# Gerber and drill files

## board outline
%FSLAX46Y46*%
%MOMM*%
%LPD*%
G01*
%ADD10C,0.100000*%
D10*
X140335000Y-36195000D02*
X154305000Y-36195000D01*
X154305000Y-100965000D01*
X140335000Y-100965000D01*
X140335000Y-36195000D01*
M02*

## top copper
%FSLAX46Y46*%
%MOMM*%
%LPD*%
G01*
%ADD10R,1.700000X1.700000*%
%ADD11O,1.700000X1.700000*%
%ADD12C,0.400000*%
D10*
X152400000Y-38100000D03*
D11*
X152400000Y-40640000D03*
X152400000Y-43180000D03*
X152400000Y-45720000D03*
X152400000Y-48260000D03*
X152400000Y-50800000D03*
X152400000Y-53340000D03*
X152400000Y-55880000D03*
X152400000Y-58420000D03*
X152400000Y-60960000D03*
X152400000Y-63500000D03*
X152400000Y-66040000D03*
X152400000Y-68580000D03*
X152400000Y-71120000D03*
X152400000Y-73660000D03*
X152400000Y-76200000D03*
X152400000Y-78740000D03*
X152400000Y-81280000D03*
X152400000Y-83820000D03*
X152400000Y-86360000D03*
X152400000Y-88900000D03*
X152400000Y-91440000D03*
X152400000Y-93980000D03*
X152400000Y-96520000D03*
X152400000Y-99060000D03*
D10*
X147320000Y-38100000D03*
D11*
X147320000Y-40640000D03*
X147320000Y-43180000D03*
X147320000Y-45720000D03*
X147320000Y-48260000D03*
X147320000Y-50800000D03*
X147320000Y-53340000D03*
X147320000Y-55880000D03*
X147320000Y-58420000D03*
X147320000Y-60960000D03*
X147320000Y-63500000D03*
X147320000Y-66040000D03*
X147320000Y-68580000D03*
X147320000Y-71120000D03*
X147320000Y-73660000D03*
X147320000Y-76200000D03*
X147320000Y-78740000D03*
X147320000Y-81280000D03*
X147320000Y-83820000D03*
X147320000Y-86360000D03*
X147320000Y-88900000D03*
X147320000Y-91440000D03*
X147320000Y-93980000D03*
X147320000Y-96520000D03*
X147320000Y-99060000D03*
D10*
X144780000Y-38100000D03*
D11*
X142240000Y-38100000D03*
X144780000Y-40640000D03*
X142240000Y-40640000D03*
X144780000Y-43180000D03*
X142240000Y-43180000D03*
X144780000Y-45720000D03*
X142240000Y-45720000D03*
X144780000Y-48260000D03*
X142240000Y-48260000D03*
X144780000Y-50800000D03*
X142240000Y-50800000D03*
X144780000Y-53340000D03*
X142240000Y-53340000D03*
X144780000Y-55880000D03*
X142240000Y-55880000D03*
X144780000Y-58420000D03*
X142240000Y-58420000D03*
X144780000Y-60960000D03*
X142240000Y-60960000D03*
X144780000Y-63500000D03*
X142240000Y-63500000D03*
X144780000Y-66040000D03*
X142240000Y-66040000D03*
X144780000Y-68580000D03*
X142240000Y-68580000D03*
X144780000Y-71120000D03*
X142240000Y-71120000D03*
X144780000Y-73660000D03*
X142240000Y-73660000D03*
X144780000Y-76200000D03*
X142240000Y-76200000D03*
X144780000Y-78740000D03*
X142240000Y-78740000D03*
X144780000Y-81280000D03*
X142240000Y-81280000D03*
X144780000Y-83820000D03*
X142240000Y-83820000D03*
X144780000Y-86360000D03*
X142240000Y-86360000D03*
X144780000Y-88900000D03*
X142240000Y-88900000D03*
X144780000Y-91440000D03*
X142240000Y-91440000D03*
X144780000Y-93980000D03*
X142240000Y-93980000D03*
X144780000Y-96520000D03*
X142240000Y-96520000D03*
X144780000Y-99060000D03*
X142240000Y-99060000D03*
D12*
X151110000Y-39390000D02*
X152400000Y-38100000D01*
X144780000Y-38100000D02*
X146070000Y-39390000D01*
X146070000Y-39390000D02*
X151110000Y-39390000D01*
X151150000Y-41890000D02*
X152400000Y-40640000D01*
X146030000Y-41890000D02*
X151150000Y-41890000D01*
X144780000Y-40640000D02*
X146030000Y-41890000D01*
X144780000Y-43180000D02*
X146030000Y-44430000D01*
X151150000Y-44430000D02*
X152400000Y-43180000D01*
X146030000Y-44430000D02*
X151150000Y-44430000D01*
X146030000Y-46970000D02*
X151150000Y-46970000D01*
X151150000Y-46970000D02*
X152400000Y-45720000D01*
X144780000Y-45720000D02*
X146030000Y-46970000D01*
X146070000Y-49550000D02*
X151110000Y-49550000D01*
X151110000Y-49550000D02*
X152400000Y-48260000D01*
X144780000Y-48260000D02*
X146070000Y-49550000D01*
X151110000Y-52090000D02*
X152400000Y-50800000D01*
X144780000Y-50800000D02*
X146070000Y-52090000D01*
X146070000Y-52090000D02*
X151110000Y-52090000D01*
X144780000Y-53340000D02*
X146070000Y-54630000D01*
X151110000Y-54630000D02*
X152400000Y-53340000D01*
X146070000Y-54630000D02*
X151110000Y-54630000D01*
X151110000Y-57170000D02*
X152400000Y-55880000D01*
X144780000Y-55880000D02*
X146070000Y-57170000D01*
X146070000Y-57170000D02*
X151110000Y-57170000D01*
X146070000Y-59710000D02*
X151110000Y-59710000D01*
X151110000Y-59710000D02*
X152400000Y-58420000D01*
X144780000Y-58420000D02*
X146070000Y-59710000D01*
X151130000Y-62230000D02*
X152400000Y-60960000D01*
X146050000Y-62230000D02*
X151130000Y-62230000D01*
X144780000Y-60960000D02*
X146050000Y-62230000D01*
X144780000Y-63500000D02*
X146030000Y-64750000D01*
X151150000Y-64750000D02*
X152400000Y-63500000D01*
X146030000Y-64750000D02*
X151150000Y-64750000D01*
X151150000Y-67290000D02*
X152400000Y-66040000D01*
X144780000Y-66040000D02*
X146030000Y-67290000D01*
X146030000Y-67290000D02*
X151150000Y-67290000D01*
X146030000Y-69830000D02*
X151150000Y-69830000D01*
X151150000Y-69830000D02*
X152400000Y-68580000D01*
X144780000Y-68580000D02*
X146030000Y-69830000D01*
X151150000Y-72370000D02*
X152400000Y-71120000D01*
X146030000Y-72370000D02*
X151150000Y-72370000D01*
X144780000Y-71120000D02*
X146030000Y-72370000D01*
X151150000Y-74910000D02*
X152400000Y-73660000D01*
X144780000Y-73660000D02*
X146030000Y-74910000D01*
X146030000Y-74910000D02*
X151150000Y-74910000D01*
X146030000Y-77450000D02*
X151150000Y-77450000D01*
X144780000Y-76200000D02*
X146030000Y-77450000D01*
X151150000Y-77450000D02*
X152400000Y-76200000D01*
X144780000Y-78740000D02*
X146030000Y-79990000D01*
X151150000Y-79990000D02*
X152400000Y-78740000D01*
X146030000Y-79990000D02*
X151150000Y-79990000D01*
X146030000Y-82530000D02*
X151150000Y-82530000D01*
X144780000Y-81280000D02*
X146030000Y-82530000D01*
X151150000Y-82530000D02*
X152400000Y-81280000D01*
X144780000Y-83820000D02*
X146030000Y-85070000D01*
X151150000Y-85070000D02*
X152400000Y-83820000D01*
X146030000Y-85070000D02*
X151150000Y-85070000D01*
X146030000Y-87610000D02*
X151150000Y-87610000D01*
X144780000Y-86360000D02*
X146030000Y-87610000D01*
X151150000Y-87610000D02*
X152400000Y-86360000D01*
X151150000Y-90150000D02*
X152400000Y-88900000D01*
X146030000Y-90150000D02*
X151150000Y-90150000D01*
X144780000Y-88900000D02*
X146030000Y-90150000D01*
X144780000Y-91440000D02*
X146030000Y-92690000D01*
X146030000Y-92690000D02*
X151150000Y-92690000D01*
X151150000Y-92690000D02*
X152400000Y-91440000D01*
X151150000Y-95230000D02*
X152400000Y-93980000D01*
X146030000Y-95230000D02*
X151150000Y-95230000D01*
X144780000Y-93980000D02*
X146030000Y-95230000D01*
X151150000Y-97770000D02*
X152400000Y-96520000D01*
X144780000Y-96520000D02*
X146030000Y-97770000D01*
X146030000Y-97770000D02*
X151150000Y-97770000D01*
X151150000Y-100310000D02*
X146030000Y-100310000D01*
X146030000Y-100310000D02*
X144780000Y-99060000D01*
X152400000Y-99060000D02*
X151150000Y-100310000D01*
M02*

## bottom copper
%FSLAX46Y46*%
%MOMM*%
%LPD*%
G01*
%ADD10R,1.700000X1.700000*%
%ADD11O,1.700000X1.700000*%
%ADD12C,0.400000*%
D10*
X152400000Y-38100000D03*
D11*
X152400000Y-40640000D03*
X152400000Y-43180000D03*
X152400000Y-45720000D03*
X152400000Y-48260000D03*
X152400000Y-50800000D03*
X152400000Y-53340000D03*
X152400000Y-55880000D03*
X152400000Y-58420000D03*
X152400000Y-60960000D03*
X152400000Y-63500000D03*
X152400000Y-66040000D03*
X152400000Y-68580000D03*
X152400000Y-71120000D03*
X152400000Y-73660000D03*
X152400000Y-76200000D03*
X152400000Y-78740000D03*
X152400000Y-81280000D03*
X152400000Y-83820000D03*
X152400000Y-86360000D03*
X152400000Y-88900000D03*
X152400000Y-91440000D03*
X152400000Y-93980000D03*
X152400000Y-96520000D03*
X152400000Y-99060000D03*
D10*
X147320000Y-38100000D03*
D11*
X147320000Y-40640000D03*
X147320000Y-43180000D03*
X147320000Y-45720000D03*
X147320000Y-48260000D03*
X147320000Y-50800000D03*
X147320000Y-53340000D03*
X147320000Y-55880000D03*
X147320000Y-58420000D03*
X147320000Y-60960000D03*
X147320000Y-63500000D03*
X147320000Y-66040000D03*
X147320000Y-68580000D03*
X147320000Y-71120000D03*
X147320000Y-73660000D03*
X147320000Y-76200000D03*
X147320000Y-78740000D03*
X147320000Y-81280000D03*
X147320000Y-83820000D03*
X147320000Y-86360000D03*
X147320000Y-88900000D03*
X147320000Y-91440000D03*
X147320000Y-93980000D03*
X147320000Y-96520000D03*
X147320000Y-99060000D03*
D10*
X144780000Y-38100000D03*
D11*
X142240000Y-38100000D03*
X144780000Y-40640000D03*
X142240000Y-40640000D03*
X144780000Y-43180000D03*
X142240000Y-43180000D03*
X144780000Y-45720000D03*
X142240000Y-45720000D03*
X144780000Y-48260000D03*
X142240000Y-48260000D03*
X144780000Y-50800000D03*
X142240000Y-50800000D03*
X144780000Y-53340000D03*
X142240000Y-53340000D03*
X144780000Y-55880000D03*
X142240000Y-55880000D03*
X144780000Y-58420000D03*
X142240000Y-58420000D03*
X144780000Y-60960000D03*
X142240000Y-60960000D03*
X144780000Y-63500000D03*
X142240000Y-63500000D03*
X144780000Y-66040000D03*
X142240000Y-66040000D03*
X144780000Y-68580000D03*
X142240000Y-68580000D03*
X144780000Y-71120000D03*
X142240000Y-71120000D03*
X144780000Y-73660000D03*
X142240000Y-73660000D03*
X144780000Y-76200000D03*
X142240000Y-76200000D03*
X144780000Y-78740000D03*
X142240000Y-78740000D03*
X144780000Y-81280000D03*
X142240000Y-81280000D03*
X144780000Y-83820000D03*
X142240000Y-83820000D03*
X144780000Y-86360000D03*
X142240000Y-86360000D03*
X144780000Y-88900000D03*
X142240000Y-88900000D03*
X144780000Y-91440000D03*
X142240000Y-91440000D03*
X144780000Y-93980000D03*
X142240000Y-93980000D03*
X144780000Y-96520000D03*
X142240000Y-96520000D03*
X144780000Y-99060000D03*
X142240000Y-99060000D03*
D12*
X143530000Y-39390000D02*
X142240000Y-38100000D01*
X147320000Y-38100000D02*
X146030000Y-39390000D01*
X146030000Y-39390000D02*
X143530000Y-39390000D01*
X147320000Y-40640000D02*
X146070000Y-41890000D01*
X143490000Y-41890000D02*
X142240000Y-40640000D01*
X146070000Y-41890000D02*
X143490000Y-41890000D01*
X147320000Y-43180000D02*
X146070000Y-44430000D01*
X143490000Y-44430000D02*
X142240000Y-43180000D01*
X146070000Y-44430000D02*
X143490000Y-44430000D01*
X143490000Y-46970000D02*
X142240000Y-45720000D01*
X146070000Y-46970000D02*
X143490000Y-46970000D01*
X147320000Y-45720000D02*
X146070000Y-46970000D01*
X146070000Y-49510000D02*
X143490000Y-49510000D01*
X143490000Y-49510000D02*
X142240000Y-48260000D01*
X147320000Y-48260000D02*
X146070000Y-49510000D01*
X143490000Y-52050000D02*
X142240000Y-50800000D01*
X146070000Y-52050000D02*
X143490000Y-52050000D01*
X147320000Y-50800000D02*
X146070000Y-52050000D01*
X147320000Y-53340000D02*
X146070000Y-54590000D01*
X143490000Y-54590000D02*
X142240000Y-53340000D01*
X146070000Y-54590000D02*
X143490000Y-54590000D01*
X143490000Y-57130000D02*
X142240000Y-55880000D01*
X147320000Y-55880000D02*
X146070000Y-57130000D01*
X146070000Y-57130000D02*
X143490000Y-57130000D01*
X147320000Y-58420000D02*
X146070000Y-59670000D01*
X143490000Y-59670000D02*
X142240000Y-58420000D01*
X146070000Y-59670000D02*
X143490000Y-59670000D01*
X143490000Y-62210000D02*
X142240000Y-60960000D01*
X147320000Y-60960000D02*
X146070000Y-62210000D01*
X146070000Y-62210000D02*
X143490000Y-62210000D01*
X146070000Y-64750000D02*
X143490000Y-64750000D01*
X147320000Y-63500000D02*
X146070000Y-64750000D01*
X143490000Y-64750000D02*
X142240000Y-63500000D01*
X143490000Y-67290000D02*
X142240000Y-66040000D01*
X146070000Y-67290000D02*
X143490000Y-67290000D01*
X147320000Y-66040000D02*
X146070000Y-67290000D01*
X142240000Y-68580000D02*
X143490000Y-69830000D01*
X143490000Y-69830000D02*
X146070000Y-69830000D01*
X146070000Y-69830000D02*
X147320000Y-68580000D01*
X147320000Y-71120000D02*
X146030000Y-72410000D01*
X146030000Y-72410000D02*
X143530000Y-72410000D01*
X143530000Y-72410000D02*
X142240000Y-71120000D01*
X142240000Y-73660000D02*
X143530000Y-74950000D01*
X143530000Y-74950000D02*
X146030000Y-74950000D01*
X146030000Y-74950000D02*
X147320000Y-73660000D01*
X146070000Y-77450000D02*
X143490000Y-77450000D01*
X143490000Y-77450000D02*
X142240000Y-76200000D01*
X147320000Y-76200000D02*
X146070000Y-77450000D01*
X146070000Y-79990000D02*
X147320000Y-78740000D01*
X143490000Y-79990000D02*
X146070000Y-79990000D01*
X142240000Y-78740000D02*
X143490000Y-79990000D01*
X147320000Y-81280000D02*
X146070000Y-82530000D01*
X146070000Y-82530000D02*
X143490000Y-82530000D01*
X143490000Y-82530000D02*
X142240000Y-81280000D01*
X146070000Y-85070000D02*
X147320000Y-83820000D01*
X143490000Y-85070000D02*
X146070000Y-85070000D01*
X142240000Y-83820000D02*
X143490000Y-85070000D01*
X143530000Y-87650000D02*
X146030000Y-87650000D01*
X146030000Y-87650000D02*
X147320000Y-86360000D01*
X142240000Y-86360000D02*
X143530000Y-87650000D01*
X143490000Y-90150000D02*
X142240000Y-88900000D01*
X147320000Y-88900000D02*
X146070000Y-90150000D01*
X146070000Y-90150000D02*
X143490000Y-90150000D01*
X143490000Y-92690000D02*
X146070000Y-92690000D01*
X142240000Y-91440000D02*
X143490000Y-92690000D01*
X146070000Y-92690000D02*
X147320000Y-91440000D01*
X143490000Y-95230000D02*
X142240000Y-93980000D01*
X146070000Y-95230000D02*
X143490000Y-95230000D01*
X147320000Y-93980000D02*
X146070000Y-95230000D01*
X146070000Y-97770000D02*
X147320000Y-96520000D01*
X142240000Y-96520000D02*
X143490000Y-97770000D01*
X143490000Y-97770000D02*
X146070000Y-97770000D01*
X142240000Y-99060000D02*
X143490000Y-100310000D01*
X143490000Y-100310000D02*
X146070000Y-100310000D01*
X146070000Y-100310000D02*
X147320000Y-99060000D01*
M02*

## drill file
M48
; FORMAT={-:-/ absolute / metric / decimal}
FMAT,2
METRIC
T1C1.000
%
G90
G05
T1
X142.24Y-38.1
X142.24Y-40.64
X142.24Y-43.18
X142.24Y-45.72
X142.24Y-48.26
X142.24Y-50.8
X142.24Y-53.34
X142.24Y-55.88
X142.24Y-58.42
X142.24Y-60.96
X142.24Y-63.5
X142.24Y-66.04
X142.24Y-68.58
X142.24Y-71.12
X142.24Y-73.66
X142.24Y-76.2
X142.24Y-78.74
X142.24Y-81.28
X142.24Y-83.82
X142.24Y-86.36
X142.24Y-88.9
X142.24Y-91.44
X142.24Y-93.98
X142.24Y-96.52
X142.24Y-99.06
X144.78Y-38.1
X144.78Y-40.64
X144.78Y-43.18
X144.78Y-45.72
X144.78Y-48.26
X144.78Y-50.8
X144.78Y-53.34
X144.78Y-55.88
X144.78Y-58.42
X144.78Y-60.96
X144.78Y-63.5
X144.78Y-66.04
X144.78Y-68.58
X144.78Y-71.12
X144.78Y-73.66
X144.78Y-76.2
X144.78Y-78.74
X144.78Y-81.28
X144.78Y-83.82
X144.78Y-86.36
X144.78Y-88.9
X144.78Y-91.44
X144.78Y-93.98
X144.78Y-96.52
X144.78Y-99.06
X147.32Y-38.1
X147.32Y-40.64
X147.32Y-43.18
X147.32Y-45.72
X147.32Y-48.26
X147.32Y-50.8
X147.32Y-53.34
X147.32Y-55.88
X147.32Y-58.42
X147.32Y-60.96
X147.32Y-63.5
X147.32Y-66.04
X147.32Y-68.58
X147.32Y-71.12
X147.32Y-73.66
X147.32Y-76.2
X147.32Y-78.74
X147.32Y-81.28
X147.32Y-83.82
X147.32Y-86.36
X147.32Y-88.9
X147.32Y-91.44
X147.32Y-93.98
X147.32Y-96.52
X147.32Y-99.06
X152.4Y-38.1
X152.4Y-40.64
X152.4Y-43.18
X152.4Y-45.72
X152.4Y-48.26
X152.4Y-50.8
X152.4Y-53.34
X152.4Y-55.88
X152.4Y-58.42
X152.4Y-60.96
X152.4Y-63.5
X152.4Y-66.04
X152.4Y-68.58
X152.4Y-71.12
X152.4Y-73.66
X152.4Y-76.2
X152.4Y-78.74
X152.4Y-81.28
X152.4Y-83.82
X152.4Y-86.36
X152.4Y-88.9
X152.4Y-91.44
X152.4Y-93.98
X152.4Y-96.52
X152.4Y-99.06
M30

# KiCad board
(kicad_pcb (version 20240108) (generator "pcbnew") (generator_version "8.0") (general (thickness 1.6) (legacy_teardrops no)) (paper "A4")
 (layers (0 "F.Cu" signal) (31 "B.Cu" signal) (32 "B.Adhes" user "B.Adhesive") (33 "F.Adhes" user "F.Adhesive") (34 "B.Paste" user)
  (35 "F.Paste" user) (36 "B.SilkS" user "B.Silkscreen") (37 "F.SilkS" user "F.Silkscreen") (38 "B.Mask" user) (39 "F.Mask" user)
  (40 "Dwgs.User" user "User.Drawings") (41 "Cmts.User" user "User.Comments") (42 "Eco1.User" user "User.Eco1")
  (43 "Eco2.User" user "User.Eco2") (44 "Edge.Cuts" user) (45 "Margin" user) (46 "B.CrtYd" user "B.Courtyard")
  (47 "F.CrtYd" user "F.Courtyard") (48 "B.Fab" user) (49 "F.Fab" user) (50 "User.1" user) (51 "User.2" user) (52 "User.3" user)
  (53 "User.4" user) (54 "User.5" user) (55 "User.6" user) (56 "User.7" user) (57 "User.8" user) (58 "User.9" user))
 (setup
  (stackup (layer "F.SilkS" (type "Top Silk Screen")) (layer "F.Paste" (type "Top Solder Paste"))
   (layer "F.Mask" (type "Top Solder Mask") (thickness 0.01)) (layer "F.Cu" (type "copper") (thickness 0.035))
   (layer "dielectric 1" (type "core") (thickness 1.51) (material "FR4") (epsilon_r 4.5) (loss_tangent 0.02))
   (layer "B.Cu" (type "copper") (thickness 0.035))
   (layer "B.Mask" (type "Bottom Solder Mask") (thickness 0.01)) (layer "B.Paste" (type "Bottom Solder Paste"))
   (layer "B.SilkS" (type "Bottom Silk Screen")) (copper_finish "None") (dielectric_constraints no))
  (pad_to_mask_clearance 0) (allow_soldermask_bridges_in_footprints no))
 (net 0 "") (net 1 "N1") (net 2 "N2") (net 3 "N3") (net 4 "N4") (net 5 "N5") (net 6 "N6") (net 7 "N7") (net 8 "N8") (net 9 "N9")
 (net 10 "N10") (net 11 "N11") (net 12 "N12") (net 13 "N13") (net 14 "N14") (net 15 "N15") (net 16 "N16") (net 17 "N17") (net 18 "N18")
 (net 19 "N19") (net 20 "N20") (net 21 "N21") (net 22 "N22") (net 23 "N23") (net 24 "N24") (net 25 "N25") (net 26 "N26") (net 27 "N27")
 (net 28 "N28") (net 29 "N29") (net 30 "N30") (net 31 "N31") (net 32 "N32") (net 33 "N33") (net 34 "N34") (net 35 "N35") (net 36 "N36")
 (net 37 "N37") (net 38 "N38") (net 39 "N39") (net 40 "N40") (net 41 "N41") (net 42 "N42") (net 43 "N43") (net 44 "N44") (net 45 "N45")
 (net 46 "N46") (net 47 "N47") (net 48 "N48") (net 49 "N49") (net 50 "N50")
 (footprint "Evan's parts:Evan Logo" (layer "F.Cu") (at 149.86 49.53 90)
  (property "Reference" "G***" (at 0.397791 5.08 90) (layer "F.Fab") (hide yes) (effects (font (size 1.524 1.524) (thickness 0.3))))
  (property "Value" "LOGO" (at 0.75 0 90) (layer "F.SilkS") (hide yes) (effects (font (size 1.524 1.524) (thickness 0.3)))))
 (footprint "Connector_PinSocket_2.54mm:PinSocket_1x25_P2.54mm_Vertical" (layer "F.Cu") (at 152.4 38.1)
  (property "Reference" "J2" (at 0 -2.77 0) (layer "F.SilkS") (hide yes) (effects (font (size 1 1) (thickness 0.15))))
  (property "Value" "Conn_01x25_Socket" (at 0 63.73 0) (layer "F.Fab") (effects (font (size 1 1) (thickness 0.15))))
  (pad "1" thru_hole rect (at 0 0) (size 1.7 1.7) (drill 1) (layers "*.Cu" "*.Mask") (remove_unused_layers no) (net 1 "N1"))
  (pad "2" thru_hole oval (at 0 2.54) (size 1.7 1.7) (drill 1) (layers "*.Cu" "*.Mask") (remove_unused_layers no) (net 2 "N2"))
  (pad "3" thru_hole oval (at 0 5.08) (size 1.7 1.7) (drill 1) (layers "*.Cu" "*.Mask") (remove_unused_layers no) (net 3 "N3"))
  (pad "4" thru_hole oval (at 0 7.62) (size 1.7 1.7) (drill 1) (layers "*.Cu" "*.Mask") (remove_unused_layers no) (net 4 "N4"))
  (pad "5" thru_hole oval (at 0 10.16) (size 1.7 1.7) (drill 1) (layers "*.Cu" "*.Mask") (remove_unused_layers no) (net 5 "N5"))
  (pad "6" thru_hole oval (at 0 12.7) (size 1.7 1.7) (drill 1) (layers "*.Cu" "*.Mask") (remove_unused_layers no) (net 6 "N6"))
  (pad "7" thru_hole oval (at 0 15.24) (size 1.7 1.7) (drill 1) (layers "*.Cu" "*.Mask") (remove_unused_layers no) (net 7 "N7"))
  (pad "8" thru_hole oval (at 0 17.78) (size 1.7 1.7) (drill 1) (layers "*.Cu" "*.Mask") (remove_unused_layers no) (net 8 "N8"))
  (pad "9" thru_hole oval (at 0 20.32) (size 1.7 1.7) (drill 1) (layers "*.Cu" "*.Mask") (remove_unused_layers no) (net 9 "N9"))
  (pad "10" thru_hole oval (at 0 22.86) (size 1.7 1.7) (drill 1) (layers "*.Cu" "*.Mask") (remove_unused_layers no) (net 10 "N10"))
  (pad "11" thru_hole oval (at 0 25.4) (size 1.7 1.7) (drill 1) (layers "*.Cu" "*.Mask") (remove_unused_layers no) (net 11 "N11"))
  (pad "12" thru_hole oval (at 0 27.94) (size 1.7 1.7) (drill 1) (layers "*.Cu" "*.Mask") (remove_unused_layers no) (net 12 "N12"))
  (pad "13" thru_hole oval (at 0 30.48) (size 1.7 1.7) (drill 1) (layers "*.Cu" "*.Mask") (remove_unused_layers no) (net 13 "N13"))
  (pad "14" thru_hole oval (at 0 33.02) (size 1.7 1.7) (drill 1) (layers "*.Cu" "*.Mask") (remove_unused_layers no) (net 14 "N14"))
  (pad "15" thru_hole oval (at 0 35.56) (size 1.7 1.7) (drill 1) (layers "*.Cu" "*.Mask") (remove_unused_layers no) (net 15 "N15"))
  (pad "16" thru_hole oval (at 0 38.1) (size 1.7 1.7) (drill 1) (layers "*.Cu" "*.Mask") (remove_unused_layers no) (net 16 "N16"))
  (pad "17" thru_hole oval (at 0 40.64) (size 1.7 1.7) (drill 1) (layers "*.Cu" "*.Mask") (remove_unused_layers no) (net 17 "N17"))
  (pad "18" thru_hole oval (at 0 43.18) (size 1.7 1.7) (drill 1) (layers "*.Cu" "*.Mask") (remove_unused_layers no) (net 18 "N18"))
  (pad "19" thru_hole oval (at 0 45.72) (size 1.7 1.7) (drill 1) (layers "*.Cu" "*.Mask") (remove_unused_layers no) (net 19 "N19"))
  (pad "20" thru_hole oval (at 0 48.26) (size 1.7 1.7) (drill 1) (layers "*.Cu" "*.Mask") (remove_unused_layers no) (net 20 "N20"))
  (pad "21" thru_hole oval (at 0 50.8) (size 1.7 1.7) (drill 1) (layers "*.Cu" "*.Mask") (remove_unused_layers no) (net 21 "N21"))
  (pad "22" thru_hole oval (at 0 53.34) (size 1.7 1.7) (drill 1) (layers "*.Cu" "*.Mask") (remove_unused_layers no) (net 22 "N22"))
  (pad "23" thru_hole oval (at 0 55.88) (size 1.7 1.7) (drill 1) (layers "*.Cu" "*.Mask") (remove_unused_layers no) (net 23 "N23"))
  (pad "24" thru_hole oval (at 0 58.42) (size 1.7 1.7) (drill 1) (layers "*.Cu" "*.Mask") (remove_unused_layers no) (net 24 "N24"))
  (pad "25" thru_hole oval (at 0 60.96) (size 1.7 1.7) (drill 1) (layers "*.Cu" "*.Mask") (remove_unused_layers no) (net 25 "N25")))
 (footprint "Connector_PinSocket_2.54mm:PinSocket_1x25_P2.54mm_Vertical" (layer "F.Cu") (at 147.32 38.1)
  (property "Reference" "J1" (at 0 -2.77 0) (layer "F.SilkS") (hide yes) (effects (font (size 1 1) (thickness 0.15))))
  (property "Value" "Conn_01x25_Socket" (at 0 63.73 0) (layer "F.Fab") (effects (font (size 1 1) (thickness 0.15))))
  (pad "1" thru_hole rect (at 0 0) (size 1.7 1.7) (drill 1) (layers "*.Cu" "*.Mask") (remove_unused_layers no) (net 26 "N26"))
  (pad "2" thru_hole oval (at 0 2.54) (size 1.7 1.7) (drill 1) (layers "*.Cu" "*.Mask") (remove_unused_layers no) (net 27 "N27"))
  (pad "3" thru_hole oval (at 0 5.08) (size 1.7 1.7) (drill 1) (layers "*.Cu" "*.Mask") (remove_unused_layers no) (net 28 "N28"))
  (pad "4" thru_hole oval (at 0 7.62) (size 1.7 1.7) (drill 1) (layers "*.Cu" "*.Mask") (remove_unused_layers no) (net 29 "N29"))
  (pad "5" thru_hole oval (at 0 10.16) (size 1.7 1.7) (drill 1) (layers "*.Cu" "*.Mask") (remove_unused_layers no) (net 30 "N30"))
  (pad "6" thru_hole oval (at 0 12.7) (size 1.7 1.7) (drill 1) (layers "*.Cu" "*.Mask") (remove_unused_layers no) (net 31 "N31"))
  (pad "7" thru_hole oval (at 0 15.24) (size 1.7 1.7) (drill 1) (layers "*.Cu" "*.Mask") (remove_unused_layers no) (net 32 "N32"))
  (pad "8" thru_hole oval (at 0 17.78) (size 1.7 1.7) (drill 1) (layers "*.Cu" "*.Mask") (remove_unused_layers no) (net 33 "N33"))
  (pad "9" thru_hole oval (at 0 20.32) (size 1.7 1.7) (drill 1) (layers "*.Cu" "*.Mask") (remove_unused_layers no) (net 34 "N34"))
  (pad "10" thru_hole oval (at 0 22.86) (size 1.7 1.7) (drill 1) (layers "*.Cu" "*.Mask") (remove_unused_layers no) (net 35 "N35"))
  (pad "11" thru_hole oval (at 0 25.4) (size 1.7 1.7) (drill 1) (layers "*.Cu" "*.Mask") (remove_unused_layers no) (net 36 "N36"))
  (pad "12" thru_hole oval (at 0 27.94) (size 1.7 1.7) (drill 1) (layers "*.Cu" "*.Mask") (remove_unused_layers no) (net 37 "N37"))
  (pad "13" thru_hole oval (at 0 30.48) (size 1.7 1.7) (drill 1) (layers "*.Cu" "*.Mask") (remove_unused_layers no) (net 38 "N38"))
  (pad "14" thru_hole oval (at 0 33.02) (size 1.7 1.7) (drill 1) (layers "*.Cu" "*.Mask") (remove_unused_layers no) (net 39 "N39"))
  (pad "15" thru_hole oval (at 0 35.56) (size 1.7 1.7) (drill 1) (layers "*.Cu" "*.Mask") (remove_unused_layers no) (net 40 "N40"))
  (pad "16" thru_hole oval (at 0 38.1) (size 1.7 1.7) (drill 1) (layers "*.Cu" "*.Mask") (remove_unused_layers no) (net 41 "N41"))
  (pad "17" thru_hole oval (at 0 40.64) (size 1.7 1.7) (drill 1) (layers "*.Cu" "*.Mask") (remove_unused_layers no) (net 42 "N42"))
  (pad "18" thru_hole oval (at 0 43.18) (size 1.7 1.7) (drill 1) (layers "*.Cu" "*.Mask") (remove_unused_layers no) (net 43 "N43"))
  (pad "19" thru_hole oval (at 0 45.72) (size 1.7 1.7) (drill 1) (layers "*.Cu" "*.Mask") (remove_unused_layers no) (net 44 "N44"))
  (pad "20" thru_hole oval (at 0 48.26) (size 1.7 1.7) (drill 1) (layers "*.Cu" "*.Mask") (remove_unused_layers no) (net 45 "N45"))
  (pad "21" thru_hole oval (at 0 50.8) (size 1.7 1.7) (drill 1) (layers "*.Cu" "*.Mask") (remove_unused_layers no) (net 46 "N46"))
  (pad "22" thru_hole oval (at 0 53.34) (size 1.7 1.7) (drill 1) (layers "*.Cu" "*.Mask") (remove_unused_layers no) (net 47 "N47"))
  (pad "23" thru_hole oval (at 0 55.88) (size 1.7 1.7) (drill 1) (layers "*.Cu" "*.Mask") (remove_unused_layers no) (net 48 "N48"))
  (pad "24" thru_hole oval (at 0 58.42) (size 1.7 1.7) (drill 1) (layers "*.Cu" "*.Mask") (remove_unused_layers no) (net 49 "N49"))
  (pad "25" thru_hole oval (at 0 60.96) (size 1.7 1.7) (drill 1) (layers "*.Cu" "*.Mask") (remove_unused_layers no) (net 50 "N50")))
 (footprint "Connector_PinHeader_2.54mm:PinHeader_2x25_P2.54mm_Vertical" (layer "B.Cu") (at 144.78 38.1 180)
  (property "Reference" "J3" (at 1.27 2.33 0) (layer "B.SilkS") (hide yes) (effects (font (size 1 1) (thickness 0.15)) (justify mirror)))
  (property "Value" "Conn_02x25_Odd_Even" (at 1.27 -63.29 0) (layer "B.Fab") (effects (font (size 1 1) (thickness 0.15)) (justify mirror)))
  (pad "1" thru_hole rect (at 0 0 180) (size 1.7 1.7) (drill 1) (layers "*.Cu" "*.Mask") (remove_unused_layers no) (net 1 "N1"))
  (pad "2" thru_hole oval (at 2.54 0 180) (size 1.7 1.7) (drill 1) (layers "*.Cu" "*.Mask") (remove_unused_layers no) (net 26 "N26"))
  (pad "3" thru_hole oval (at 0 -2.54 180) (size 1.7 1.7) (drill 1) (layers "*.Cu" "*.Mask") (remove_unused_layers no) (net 2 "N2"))
  (pad "4" thru_hole oval (at 2.54 -2.54 180) (size 1.7 1.7) (drill 1) (layers "*.Cu" "*.Mask") (remove_unused_layers no) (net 27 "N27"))
  (pad "5" thru_hole oval (at 0 -5.08 180) (size 1.7 1.7) (drill 1) (layers "*.Cu" "*.Mask") (remove_unused_layers no) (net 3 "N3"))
  (pad "6" thru_hole oval (at 2.54 -5.08 180) (size 1.7 1.7) (drill 1) (layers "*.Cu" "*.Mask") (remove_unused_layers no) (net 28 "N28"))
  (pad "7" thru_hole oval (at 0 -7.62 180) (size 1.7 1.7) (drill 1) (layers "*.Cu" "*.Mask") (remove_unused_layers no) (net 4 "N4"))
  (pad "8" thru_hole oval (at 2.54 -7.62 180) (size 1.7 1.7) (drill 1) (layers "*.Cu" "*.Mask") (remove_unused_layers no) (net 29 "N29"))
  (pad "9" thru_hole oval (at 0 -10.16 180) (size 1.7 1.7) (drill 1) (layers "*.Cu" "*.Mask") (remove_unused_layers no) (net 5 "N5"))
  (pad "10" thru_hole oval (at 2.54 -10.16 180) (size 1.7 1.7) (drill 1) (layers "*.Cu" "*.Mask") (remove_unused_layers no) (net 30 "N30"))
  (pad "11" thru_hole oval (at 0 -12.7 180) (size 1.7 1.7) (drill 1) (layers "*.Cu" "*.Mask") (remove_unused_layers no) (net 6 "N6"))
  (pad "12" thru_hole oval (at 2.54 -12.7 180) (size 1.7 1.7) (drill 1) (layers "*.Cu" "*.Mask") (remove_unused_layers no) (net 31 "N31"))
  (pad "13" thru_hole oval (at 0 -15.24 180) (size 1.7 1.7) (drill 1) (layers "*.Cu" "*.Mask") (remove_unused_layers no) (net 7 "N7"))
  (pad "14" thru_hole oval (at 2.54 -15.24 180) (size 1.7 1.7) (drill 1) (layers "*.Cu" "*.Mask") (remove_unused_layers no) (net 32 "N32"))
  (pad "15" thru_hole oval (at 0 -17.78 180) (size 1.7 1.7) (drill 1) (layers "*.Cu" "*.Mask") (remove_unused_layers no) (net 8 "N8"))
  (pad "16" thru_hole oval (at 2.54 -17.78 180) (size 1.7 1.7) (drill 1) (layers "*.Cu" "*.Mask") (remove_unused_layers no) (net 33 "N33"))
  (pad "17" thru_hole oval (at 0 -20.32 180) (size 1.7 1.7) (drill 1) (layers "*.Cu" "*.Mask") (remove_unused_layers no) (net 9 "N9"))
  (pad "18" thru_hole oval (at 2.54 -20.32 180) (size 1.7 1.7) (drill 1) (layers "*.Cu" "*.Mask") (remove_unused_layers no) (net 34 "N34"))
  (pad "19" thru_hole oval (at 0 -22.86 180) (size 1.7 1.7) (drill 1) (layers "*.Cu" "*.Mask") (remove_unused_layers no) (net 10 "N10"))
  (pad "20" thru_hole oval (at 2.54 -22.86 180) (size 1.7 1.7) (drill 1) (layers "*.Cu" "*.Mask") (remove_unused_layers no) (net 35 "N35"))
  (pad "21" thru_hole oval (at 0 -25.4 180) (size 1.7 1.7) (drill 1) (layers "*.Cu" "*.Mask") (remove_unused_layers no) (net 11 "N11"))
  (pad "22" thru_hole oval (at 2.54 -25.4 180) (size 1.7 1.7) (drill 1) (layers "*.Cu" "*.Mask") (remove_unused_layers no) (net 36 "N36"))
  (pad "23" thru_hole oval (at 0 -27.94 180) (size 1.7 1.7) (drill 1) (layers "*.Cu" "*.Mask") (remove_unused_layers no) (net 12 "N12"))
  (pad "24" thru_hole oval (at 2.54 -27.94 180) (size 1.7 1.7) (drill 1) (layers "*.Cu" "*.Mask") (remove_unused_layers no) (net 37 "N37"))
  (pad "25" thru_hole oval (at 0 -30.48 180) (size 1.7 1.7) (drill 1) (layers "*.Cu" "*.Mask") (remove_unused_layers no) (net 13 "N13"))
  (pad "26" thru_hole oval (at 2.54 -30.48 180) (size 1.7 1.7) (drill 1) (layers "*.Cu" "*.Mask") (remove_unused_layers no) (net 38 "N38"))
  (pad "27" thru_hole oval (at 0 -33.02 180) (size 1.7 1.7) (drill 1) (layers "*.Cu" "*.Mask") (remove_unused_layers no) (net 14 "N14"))
  (pad "28" thru_hole oval (at 2.54 -33.02 180) (size 1.7 1.7) (drill 1) (layers "*.Cu" "*.Mask") (remove_unused_layers no) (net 39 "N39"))
  (pad "29" thru_hole oval (at 0 -35.56 180) (size 1.7 1.7) (drill 1) (layers "*.Cu" "*.Mask") (remove_unused_layers no) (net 15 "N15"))
  (pad "30" thru_hole oval (at 2.54 -35.56 180) (size 1.7 1.7) (drill 1) (layers "*.Cu" "*.Mask") (remove_unused_layers no) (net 40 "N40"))
  (pad "31" thru_hole oval (at 0 -38.1 180) (size 1.7 1.7) (drill 1) (layers "*.Cu" "*.Mask") (remove_unused_layers no) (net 16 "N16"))
  (pad "32" thru_hole oval (at 2.54 -38.1 180) (size 1.7 1.7) (drill 1) (layers "*.Cu" "*.Mask") (remove_unused_layers no) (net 41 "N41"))
  (pad "33" thru_hole oval (at 0 -40.64 180) (size 1.7 1.7) (drill 1) (layers "*.Cu" "*.Mask") (remove_unused_layers no) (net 17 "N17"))
  (pad "34" thru_hole oval (at 2.54 -40.64 180) (size 1.7 1.7) (drill 1) (layers "*.Cu" "*.Mask") (remove_unused_layers no) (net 42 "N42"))
  (pad "35" thru_hole oval (at 0 -43.18 180) (size 1.7 1.7) (drill 1) (layers "*.Cu" "*.Mask") (remove_unused_layers no) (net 18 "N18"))
  (pad "36" thru_hole oval (at 2.54 -43.18 180) (size 1.7 1.7) (drill 1) (layers "*.Cu" "*.Mask") (remove_unused_layers no) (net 43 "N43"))
  (pad "37" thru_hole oval (at 0 -45.72 180) (size 1.7 1.7) (drill 1) (layers "*.Cu" "*.Mask") (remove_unused_layers no) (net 19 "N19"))
  (pad "38" thru_hole oval (at 2.54 -45.72 180) (size 1.7 1.7) (drill 1) (layers "*.Cu" "*.Mask") (remove_unused_layers no) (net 44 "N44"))
  (pad "39" thru_hole oval (at 0 -48.26 180) (size 1.7 1.7) (drill 1) (layers "*.Cu" "*.Mask") (remove_unused_layers no) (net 20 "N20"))
  (pad "40" thru_hole oval (at 2.54 -48.26 180) (size 1.7 1.7) (drill 1) (layers "*.Cu" "*.Mask") (remove_unused_layers no) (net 45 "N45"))
  (pad "41" thru_hole oval (at 0 -50.8 180) (size 1.7 1.7) (drill 1) (layers "*.Cu" "*.Mask") (remove_unused_layers no) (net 21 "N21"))
  (pad "42" thru_hole oval (at 2.54 -50.8 180) (size 1.7 1.7) (drill 1) (layers "*.Cu" "*.Mask") (remove_unused_layers no) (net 46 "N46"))
  (pad "43" thru_hole oval (at 0 -53.34 180) (size 1.7 1.7) (drill 1) (layers "*.Cu" "*.Mask") (remove_unused_layers no) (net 22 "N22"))
  (pad "44" thru_hole oval (at 2.54 -53.34 180) (size 1.7 1.7) (drill 1) (layers "*.Cu" "*.Mask") (remove_unused_layers no) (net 47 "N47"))
  (pad "45" thru_hole oval (at 0 -55.88 180) (size 1.7 1.7) (drill 1) (layers "*.Cu" "*.Mask") (remove_unused_layers no) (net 23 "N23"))
  (pad "46" thru_hole oval (at 2.54 -55.88 180) (size 1.7 1.7) (drill 1) (layers "*.Cu" "*.Mask") (remove_unused_layers no) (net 48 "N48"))
  (pad "47" thru_hole oval (at 0 -58.42 180) (size 1.7 1.7) (drill 1) (layers "*.Cu" "*.Mask") (remove_unused_layers no) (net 24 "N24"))
  (pad "48" thru_hole oval (at 2.54 -58.42 180) (size 1.7 1.7) (drill 1) (layers "*.Cu" "*.Mask") (remove_unused_layers no) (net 49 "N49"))
  (pad "49" thru_hole oval (at 0 -60.96 180) (size 1.7 1.7) (drill 1) (layers "*.Cu" "*.Mask") (remove_unused_layers no) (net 25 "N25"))
  (pad "50" thru_hole oval (at 2.54 -60.96 180) (size 1.7 1.7) (drill 1) (layers "*.Cu" "*.Mask") (remove_unused_layers no) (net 50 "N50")))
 (gr_rect (start 140.335 36.195) (end 154.305 100.965) (stroke (width 0.1) (type default)) (fill none) (layer "Edge.Cuts"))
 (segment (start 143.53 39.39) (end 142.24 38.1) (width 0.4) (layer "B.Cu") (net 26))
 (segment (start 147.32 38.1) (end 146.03 39.39) (width 0.4) (layer "B.Cu") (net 26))
 (segment (start 146.03 39.39) (end 143.53 39.39) (width 0.4) (layer "B.Cu") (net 26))
 (segment (start 147.32 40.64) (end 146.07 41.89) (width 0.4) (layer "B.Cu") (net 27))
 (segment (start 143.49 41.89) (end 142.24 40.64) (width 0.4) (layer "B.Cu") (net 27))
 (segment (start 146.07 41.89) (end 143.49 41.89) (width 0.4) (layer "B.Cu") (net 27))
 (segment (start 147.32 43.18) (end 146.07 44.43) (width 0.4) (layer "B.Cu") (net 28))
 (segment (start 143.49 44.43) (end 142.24 43.18) (width 0.4) (layer "B.Cu") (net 28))
 (segment (start 146.07 44.43) (end 143.49 44.43) (width 0.4) (layer "B.Cu") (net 28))
 (segment (start 143.49 46.97) (end 142.24 45.72) (width 0.4) (layer "B.Cu") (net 29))
 (segment (start 146.07 46.97) (end 143.49 46.97) (width 0.4) (layer "B.Cu") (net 29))
 (segment (start 147.32 45.72) (end 146.07 46.97) (width 0.4) (layer "B.Cu") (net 29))
 (segment (start 146.07 49.51) (end 143.49 49.51) (width 0.4) (layer "B.Cu") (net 30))
 (segment (start 143.49 49.51) (end 142.24 48.26) (width 0.4) (layer "B.Cu") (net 30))
 (segment (start 147.32 48.26) (end 146.07 49.51) (width 0.4) (layer "B.Cu") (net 30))
 (segment (start 143.49 52.05) (end 142.24 50.8) (width 0.4) (layer "B.Cu") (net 31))
 (segment (start 146.07 52.05) (end 143.49 52.05) (width 0.4) (layer "B.Cu") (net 31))
 (segment (start 147.32 50.8) (end 146.07 52.05) (width 0.4) (layer "B.Cu") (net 31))
 (segment (start 147.32 53.34) (end 146.07 54.59) (width 0.4) (layer "B.Cu") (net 32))
 (segment (start 143.49 54.59) (end 142.24 53.34) (width 0.4) (layer "B.Cu") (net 32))
 (segment (start 146.07 54.59) (end 143.49 54.59) (width 0.4) (layer "B.Cu") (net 32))
 (segment (start 143.49 57.13) (end 142.24 55.88) (width 0.4) (layer "B.Cu") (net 33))
 (segment (start 147.32 55.88) (end 146.07 57.13) (width 0.4) (layer "B.Cu") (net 33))
 (segment (start 146.07 57.13) (end 143.49 57.13) (width 0.4) (layer "B.Cu") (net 33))
 (segment (start 147.32 58.42) (end 146.07 59.67) (width 0.4) (layer "B.Cu") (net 34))
 (segment (start 143.49 59.67) (end 142.24 58.42) (width 0.4) (layer "B.Cu") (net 34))
 (segment (start 146.07 59.67) (end 143.49 59.67) (width 0.4) (layer "B.Cu") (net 34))
 (segment (start 143.49 62.21) (end 142.24 60.96) (width 0.4) (layer "B.Cu") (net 35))
 (segment (start 147.32 60.96) (end 146.07 62.21) (width 0.4) (layer "B.Cu") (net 35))
 (segment (start 146.07 62.21) (end 143.49 62.21) (width 0.4) (layer "B.Cu") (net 35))
 (segment (start 146.07 64.75) (end 143.49 64.75) (width 0.4) (layer "B.Cu") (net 36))
 (segment (start 147.32 63.5) (end 146.07 64.75) (width 0.4) (layer "B.Cu") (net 36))
 (segment (start 143.49 64.75) (end 142.24 63.5) (width 0.4) (layer "B.Cu") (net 36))
 (segment (start 143.49 67.29) (end 142.24 66.04) (width 0.4) (layer "B.Cu") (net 37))
 (segment (start 146.07 67.29) (end 143.49 67.29) (width 0.4) (layer "B.Cu") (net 37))
 (segment (start 147.32 66.04) (end 146.07 67.29) (width 0.4) (layer "B.Cu") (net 37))
 (segment (start 142.24 68.58) (end 143.49 69.83) (width 0.4) (layer "B.Cu") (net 38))
 (segment (start 143.49 69.83) (end 146.07 69.83) (width 0.4) (layer "B.Cu") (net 38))
 (segment (start 146.07 69.83) (end 147.32 68.58) (width 0.4) (layer "B.Cu") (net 38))
 (segment (start 147.32 71.12) (end 146.03 72.41) (width 0.4) (layer "B.Cu") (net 39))
 (segment (start 146.03 72.41) (end 143.53 72.41) (width 0.4) (layer "B.Cu") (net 39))
 (segment (start 143.53 72.41) (end 142.24 71.12) (width 0.4) (layer "B.Cu") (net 39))
 (segment (start 142.24 73.66) (end 143.53 74.95) (width 0.4) (layer "B.Cu") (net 40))
 (segment (start 143.53 74.95) (end 146.03 74.95) (width 0.4) (layer "B.Cu") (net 40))
 (segment (start 146.03 74.95) (end 147.32 73.66) (width 0.4) (layer "B.Cu") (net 40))
 (segment (start 146.07 77.45) (end 143.49 77.45) (width 0.4) (layer "B.Cu") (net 41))
 (segment (start 143.49 77.45) (end 142.24 76.2) (width 0.4) (layer "B.Cu") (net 41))
 (segment (start 147.32 76.2) (end 146.07 77.45) (width 0.4) (layer "B.Cu") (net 41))
 (segment (start 146.07 79.99) (end 147.32 78.74) (width 0.4) (layer "B.Cu") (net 42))
 (segment (start 143.49 79.99) (end 146.07 79.99) (width 0.4) (layer "B.Cu") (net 42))
 (segment (start 142.24 78.74) (end 143.49 79.99) (width 0.4) (layer "B.Cu") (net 42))
 (segment (start 147.32 81.28) (end 146.07 82.53) (width 0.4) (layer "B.Cu") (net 43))
 (segment (start 146.07 82.53) (end 143.49 82.53) (width 0.4) (layer "B.Cu") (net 43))
 (segment (start 143.49 82.53) (end 142.24 81.28) (width 0.4) (layer "B.Cu") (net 43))
 (segment (start 146.07 85.07) (end 147.32 83.82) (width 0.4) (layer "B.Cu") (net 44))
 (segment (start 143.49 85.07) (end 146.07 85.07) (width 0.4) (layer "B.Cu") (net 44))
 (segment (start 142.24 83.82) (end 143.49 85.07) (width 0.4) (layer "B.Cu") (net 44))
 (segment (start 143.53 87.65) (end 146.03 87.65) (width 0.4) (layer "B.Cu") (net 45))
 (segment (start 146.03 87.65) (end 147.32 86.36) (width 0.4) (layer "B.Cu") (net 45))
 (segment (start 142.24 86.36) (end 143.53 87.65) (width 0.4) (layer "B.Cu") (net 45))
 (segment (start 143.49 90.15) (end 142.24 88.9) (width 0.4) (layer "B.Cu") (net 46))
 (segment (start 147.32 88.9) (end 146.07 90.15) (width 0.4) (layer "B.Cu") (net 46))
 (segment (start 146.07 90.15) (end 143.49 90.15) (width 0.4) (layer "B.Cu") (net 46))
 (segment (start 143.49 92.69) (end 146.07 92.69) (width 0.4) (layer "B.Cu") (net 47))
 (segment (start 142.24 91.44) (end 143.49 92.69) (width 0.4) (layer "B.Cu") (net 47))
 (segment (start 146.07 92.69) (end 147.32 91.44) (width 0.4) (layer "B.Cu") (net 47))
 (segment (start 143.49 95.23) (end 142.24 93.98) (width 0.4) (layer "B.Cu") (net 48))
 (segment (start 146.07 95.23) (end 143.49 95.23) (width 0.4) (layer "B.Cu") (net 48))
 (segment (start 147.32 93.98) (end 146.07 95.23) (width 0.4) (layer "B.Cu") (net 48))
 (segment (start 146.07 97.77) (end 147.32 96.52) (width 0.4) (layer "B.Cu") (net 49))
 (segment (start 142.24 96.52) (end 143.49 97.77) (width 0.4) (layer "B.Cu") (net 49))
 (segment (start 143.49 97.77) (end 146.07 97.77) (width 0.4) (layer "B.Cu") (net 49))
 (segment (start 142.24 99.06) (end 143.49 100.31) (width 0.4) (layer "B.Cu") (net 50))
 (segment (start 143.49 100.31) (end 146.07 100.31) (width 0.4) (layer "B.Cu") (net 50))
 (segment (start 146.07 100.31) (end 147.32 99.06) (width 0.4) (layer "B.Cu") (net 50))
 (segment (start 151.11 39.39) (end 152.4 38.1) (width 0.4) (layer "F.Cu") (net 1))
 (segment (start 144.78 38.1) (end 146.07 39.39) (width 0.4) (layer "F.Cu") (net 1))
 (segment (start 146.07 39.39) (end 151.11 39.39) (width 0.4) (layer "F.Cu") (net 1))
 (segment (start 151.15 41.89) (end 152.4 40.64) (width 0.4) (layer "F.Cu") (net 2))
 (segment (start 146.03 41.89) (end 151.15 41.89) (width 0.4) (layer "F.Cu") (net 2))
 (segment (start 144.78 40.64) (end 146.03 41.89) (width 0.4) (layer "F.Cu") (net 2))
 (segment (start 144.78 43.18) (end 146.03 44.43) (width 0.4) (layer "F.Cu") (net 3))
 (segment (start 151.15 44.43) (end 152.4 43.18) (width 0.4) (layer "F.Cu") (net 3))
 (segment (start 146.03 44.43) (end 151.15 44.43) (width 0.4) (layer "F.Cu") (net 3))
 (segment (start 146.03 46.97) (end 151.15 46.97) (width 0.4) (layer "F.Cu") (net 4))
 (segment (start 151.15 46.97) (end 152.4 45.72) (width 0.4) (layer "F.Cu") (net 4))
 (segment (start 144.78 45.72) (end 146.03 46.97) (width 0.4) (layer "F.Cu") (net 4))
 (segment (start 146.07 49.55) (end 151.11 49.55) (width 0.4) (layer "F.Cu") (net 5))
 (segment (start 151.11 49.55) (end 152.4 48.26) (width 0.4) (layer "F.Cu") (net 5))
 (segment (start 144.78 48.26) (end 146.07 49.55) (width 0.4) (layer "F.Cu") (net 5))
 (segment (start 151.11 52.09) (end 152.4 50.8) (width 0.4) (layer "F.Cu") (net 6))
 (segment (start 144.78 50.8) (end 146.07 52.09) (width 0.4) (layer "F.Cu") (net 6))
 (segment (start 146.07 52.09) (end 151.11 52.09) (width 0.4) (layer "F.Cu") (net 6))
 (segment (start 144.78 53.34) (end 146.07 54.63) (width 0.4) (layer "F.Cu") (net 7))
 (segment (start 151.11 54.63) (end 152.4 53.34) (width 0.4) (layer "F.Cu") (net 7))
 (segment (start 146.07 54.63) (end 151.11 54.63) (width 0.4) (layer "F.Cu") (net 7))
 (segment (start 151.11 57.17) (end 152.4 55.88) (width 0.4) (layer "F.Cu") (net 8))
 (segment (start 144.78 55.88) (end 146.07 57.17) (width 0.4) (layer "F.Cu") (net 8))
 (segment (start 146.07 57.17) (end 151.11 57.17) (width 0.4) (layer "F.Cu") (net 8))
 (segment (start 146.07 59.71) (end 151.11 59.71) (width 0.4) (layer "F.Cu") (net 9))
 (segment (start 151.11 59.71) (end 152.4 58.42) (width 0.4) (layer "F.Cu") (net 9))
 (segment (start 144.78 58.42) (end 146.07 59.71) (width 0.4) (layer "F.Cu") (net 9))
 (segment (start 151.13 62.23) (end 152.4 60.96) (width 0.4) (layer "F.Cu") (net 10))
 (segment (start 146.05 62.23) (end 151.13 62.23) (width 0.4) (layer "F.Cu") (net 10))
 (segment (start 144.78 60.96) (end 146.05 62.23) (width 0.4) (layer "F.Cu") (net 10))
 (segment (start 144.78 63.5) (end 146.03 64.75) (width 0.4) (layer "F.Cu") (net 11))
 (segment (start 151.15 64.75) (end 152.4 63.5) (width 0.4) (layer "F.Cu") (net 11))
 (segment (start 146.03 64.75) (end 151.15 64.75) (width 0.4) (layer "F.Cu") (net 11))
 (segment (start 151.15 67.29) (end 152.4 66.04) (width 0.4) (layer "F.Cu") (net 12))
 (segment (start 144.78 66.04) (end 146.03 67.29) (width 0.4) (layer "F.Cu") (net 12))
 (segment (start 146.03 67.29) (end 151.15 67.29) (width 0.4) (layer "F.Cu") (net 12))
 (segment (start 146.03 69.83) (end 151.15 69.83) (width 0.4) (layer "F.Cu") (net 13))
 (segment (start 151.15 69.83) (end 152.4 68.58) (width 0.4) (layer "F.Cu") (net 13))
 (segment (start 144.78 68.58) (end 146.03 69.83) (width 0.4) (layer "F.Cu") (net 13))
 (segment (start 151.15 72.37) (end 152.4 71.12) (width 0.4) (layer "F.Cu") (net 14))
 (segment (start 146.03 72.37) (end 151.15 72.37) (width 0.4) (layer "F.Cu") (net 14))
 (segment (start 144.78 71.12) (end 146.03 72.37) (width 0.4) (layer "F.Cu") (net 14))
 (segment (start 151.15 74.91) (end 152.4 73.66) (width 0.4) (layer "F.Cu") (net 15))
 (segment (start 144.78 73.66) (end 146.03 74.91) (width 0.4) (layer "F.Cu") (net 15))
 (segment (start 146.03 74.91) (end 151.15 74.91) (width 0.4) (layer "F.Cu") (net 15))
 (segment (start 146.03 77.45) (end 151.15 77.45) (width 0.4) (layer "F.Cu") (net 16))
 (segment (start 144.78 76.2) (end 146.03 77.45) (width 0.4) (layer "F.Cu") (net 16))
 (segment (start 151.15 77.45) (end 152.4 76.2) (width 0.4) (layer "F.Cu") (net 16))
 (segment (start 144.78 78.74) (end 146.03 79.99) (width 0.4) (layer "F.Cu") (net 17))
 (segment (start 151.15 79.99) (end 152.4 78.74) (width 0.4) (layer "F.Cu") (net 17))
 (segment (start 146.03 79.99) (end 151.15 79.99) (width 0.4) (layer "F.Cu") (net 17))
 (segment (start 146.03 82.53) (end 151.15 82.53) (width 0.4) (layer "F.Cu") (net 18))
 (segment (start 144.78 81.28) (end 146.03 82.53) (width 0.4) (layer "F.Cu") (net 18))
 (segment (start 151.15 82.53) (end 152.4 81.28) (width 0.4) (layer "F.Cu") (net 18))
 (segment (start 144.78 83.82) (end 146.03 85.07) (width 0.4) (layer "F.Cu") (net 19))
 (segment (start 151.15 85.07) (end 152.4 83.82) (width 0.4) (layer "F.Cu") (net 19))
 (segment (start 146.03 85.07) (end 151.15 85.07) (width 0.4) (layer "F.Cu") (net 19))
 (segment (start 146.03 87.61) (end 151.15 87.61) (width 0.4) (layer "F.Cu") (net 20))
 (segment (start 144.78 86.36) (end 146.03 87.61) (width 0.4) (layer "F.Cu") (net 20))
 (segment (start 151.15 87.61) (end 152.4 86.36) (width 0.4) (layer "F.Cu") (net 20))
 (segment (start 151.15 90.15) (end 152.4 88.9) (width 0.4) (layer "F.Cu") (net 21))
 (segment (start 146.03 90.15) (end 151.15 90.15) (width 0.4) (layer "F.Cu") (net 21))
 (segment (start 144.78 88.9) (end 146.03 90.15) (width 0.4) (layer "F.Cu") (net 21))
 (segment (start 144.78 91.44) (end 146.03 92.69) (width 0.4) (layer "F.Cu") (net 22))
 (segment (start 146.03 92.69) (end 151.15 92.69) (width 0.4) (layer "F.Cu") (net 22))
 (segment (start 151.15 92.69) (end 152.4 91.44) (width 0.4) (layer "F.Cu") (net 22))
 (segment (start 151.15 95.23) (end 152.4 93.98) (width 0.4) (layer "F.Cu") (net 23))
 (segment (start 146.03 95.23) (end 151.15 95.23) (width 0.4) (layer "F.Cu") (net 23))
 (segment (start 144.78 93.98) (end 146.03 95.23) (width 0.4) (layer "F.Cu") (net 23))
 (segment (start 151.15 97.77) (end 152.4 96.52) (width 0.4) (layer "F.Cu") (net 24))
 (segment (start 144.78 96.52) (end 146.03 97.77) (width 0.4) (layer "F.Cu") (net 24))
 (segment (start 146.03 97.77) (end 151.15 97.77) (width 0.4) (layer "F.Cu") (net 24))
 (segment (start 151.15 100.31) (end 146.03 100.31) (width 0.4) (layer "F.Cu") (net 25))
 (segment (start 146.03 100.31) (end 144.78 99.06) (width 0.4) (layer "F.Cu") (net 25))
 (segment (start 152.4 99.06) (end 151.15 100.31) (width 0.4) (layer "F.Cu") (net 25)))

